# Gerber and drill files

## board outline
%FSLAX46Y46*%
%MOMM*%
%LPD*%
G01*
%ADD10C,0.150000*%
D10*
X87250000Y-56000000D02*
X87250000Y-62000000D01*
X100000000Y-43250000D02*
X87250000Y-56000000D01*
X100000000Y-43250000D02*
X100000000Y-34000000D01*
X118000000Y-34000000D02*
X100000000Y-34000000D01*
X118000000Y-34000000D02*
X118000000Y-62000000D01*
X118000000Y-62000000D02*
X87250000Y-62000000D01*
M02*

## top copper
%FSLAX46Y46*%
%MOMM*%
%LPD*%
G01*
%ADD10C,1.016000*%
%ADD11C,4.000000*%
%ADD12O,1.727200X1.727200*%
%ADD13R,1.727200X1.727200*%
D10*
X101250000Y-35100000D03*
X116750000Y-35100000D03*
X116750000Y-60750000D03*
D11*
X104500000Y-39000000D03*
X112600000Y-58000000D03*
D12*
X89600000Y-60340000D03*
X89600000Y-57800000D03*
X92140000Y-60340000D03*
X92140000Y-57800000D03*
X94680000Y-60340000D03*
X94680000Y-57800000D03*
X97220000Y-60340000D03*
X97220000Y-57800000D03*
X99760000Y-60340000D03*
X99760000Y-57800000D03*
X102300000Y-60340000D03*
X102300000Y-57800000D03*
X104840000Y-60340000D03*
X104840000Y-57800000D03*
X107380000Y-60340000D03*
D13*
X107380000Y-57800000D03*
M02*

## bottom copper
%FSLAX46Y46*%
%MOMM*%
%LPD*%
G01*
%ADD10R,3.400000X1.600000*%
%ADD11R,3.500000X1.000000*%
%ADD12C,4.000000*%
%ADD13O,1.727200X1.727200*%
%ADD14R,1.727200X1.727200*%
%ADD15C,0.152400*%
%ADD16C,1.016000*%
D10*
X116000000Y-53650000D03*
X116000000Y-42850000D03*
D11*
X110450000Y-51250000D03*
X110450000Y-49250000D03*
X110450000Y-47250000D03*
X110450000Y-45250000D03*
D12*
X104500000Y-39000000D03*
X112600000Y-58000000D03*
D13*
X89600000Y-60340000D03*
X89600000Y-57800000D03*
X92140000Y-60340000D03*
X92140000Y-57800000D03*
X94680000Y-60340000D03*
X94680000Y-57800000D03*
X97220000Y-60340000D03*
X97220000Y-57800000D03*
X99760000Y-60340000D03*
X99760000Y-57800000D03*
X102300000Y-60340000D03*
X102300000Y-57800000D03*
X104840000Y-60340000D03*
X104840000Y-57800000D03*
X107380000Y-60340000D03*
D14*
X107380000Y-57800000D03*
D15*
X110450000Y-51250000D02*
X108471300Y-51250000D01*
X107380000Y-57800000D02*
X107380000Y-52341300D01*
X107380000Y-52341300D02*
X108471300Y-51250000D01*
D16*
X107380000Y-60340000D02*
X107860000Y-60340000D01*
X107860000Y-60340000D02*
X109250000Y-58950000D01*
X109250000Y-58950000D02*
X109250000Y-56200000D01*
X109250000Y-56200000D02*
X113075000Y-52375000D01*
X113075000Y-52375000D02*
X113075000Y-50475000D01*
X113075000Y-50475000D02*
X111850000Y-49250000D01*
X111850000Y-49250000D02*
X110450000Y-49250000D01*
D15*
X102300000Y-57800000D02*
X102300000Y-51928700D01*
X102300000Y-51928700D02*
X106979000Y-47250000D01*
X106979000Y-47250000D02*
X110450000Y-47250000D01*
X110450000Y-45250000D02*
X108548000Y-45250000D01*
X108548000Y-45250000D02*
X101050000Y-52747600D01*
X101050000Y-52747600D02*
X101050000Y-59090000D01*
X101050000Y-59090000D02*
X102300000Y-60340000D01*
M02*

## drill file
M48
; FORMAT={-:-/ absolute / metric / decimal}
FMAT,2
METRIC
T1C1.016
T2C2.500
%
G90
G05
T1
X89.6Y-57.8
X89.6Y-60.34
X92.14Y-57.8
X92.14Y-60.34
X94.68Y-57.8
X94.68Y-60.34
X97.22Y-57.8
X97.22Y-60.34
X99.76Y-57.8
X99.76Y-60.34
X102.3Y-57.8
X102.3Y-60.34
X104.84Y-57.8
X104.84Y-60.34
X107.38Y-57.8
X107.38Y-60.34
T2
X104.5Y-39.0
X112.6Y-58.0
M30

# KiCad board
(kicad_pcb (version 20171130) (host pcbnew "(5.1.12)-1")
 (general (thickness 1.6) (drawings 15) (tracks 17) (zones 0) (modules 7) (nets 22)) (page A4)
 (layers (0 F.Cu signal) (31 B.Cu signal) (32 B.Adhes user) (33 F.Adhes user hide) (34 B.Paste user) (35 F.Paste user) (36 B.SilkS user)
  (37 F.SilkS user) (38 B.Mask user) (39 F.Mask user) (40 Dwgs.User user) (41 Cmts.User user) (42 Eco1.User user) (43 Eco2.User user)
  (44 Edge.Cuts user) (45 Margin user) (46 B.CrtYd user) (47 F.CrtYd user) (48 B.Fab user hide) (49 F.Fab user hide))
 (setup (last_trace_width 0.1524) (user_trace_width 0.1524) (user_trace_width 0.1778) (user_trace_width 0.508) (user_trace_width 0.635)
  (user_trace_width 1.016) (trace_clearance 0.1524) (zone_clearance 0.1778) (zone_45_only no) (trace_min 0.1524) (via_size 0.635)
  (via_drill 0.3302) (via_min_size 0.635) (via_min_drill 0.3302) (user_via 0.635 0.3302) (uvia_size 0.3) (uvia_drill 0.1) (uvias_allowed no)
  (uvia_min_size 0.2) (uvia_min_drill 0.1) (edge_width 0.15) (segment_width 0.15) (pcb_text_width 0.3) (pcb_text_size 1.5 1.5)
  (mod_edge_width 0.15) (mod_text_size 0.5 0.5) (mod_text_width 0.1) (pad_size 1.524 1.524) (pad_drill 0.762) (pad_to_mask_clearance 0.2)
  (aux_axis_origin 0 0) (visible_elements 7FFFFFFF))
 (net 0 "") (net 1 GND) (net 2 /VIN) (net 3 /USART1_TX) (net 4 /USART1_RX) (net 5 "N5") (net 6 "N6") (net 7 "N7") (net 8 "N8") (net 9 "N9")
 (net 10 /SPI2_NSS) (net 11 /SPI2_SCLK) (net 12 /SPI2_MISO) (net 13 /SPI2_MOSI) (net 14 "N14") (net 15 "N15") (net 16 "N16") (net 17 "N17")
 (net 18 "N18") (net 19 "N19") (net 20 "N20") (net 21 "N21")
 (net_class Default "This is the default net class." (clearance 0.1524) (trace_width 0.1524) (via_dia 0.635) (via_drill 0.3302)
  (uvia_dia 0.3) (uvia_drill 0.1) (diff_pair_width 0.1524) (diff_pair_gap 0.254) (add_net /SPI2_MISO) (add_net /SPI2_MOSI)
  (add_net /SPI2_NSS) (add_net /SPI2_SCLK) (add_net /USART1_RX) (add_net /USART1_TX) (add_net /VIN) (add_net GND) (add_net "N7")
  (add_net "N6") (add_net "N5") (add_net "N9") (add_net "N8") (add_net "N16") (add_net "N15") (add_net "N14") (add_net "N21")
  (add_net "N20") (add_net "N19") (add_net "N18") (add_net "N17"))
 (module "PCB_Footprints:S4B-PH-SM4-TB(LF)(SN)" (layer B.Cu) (at 113.225 48.25 270)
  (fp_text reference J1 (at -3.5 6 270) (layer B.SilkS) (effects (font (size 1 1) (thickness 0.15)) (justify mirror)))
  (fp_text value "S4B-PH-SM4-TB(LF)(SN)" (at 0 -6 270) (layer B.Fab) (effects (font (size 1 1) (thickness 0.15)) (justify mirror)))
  (pad "" smd rect (at 5.4 -2.775 270) (size 1.6 3.4) (layers B.Cu B.Paste B.Mask))
  (pad "" smd rect (at -5.4 -2.775 270) (size 1.6 3.4) (layers B.Cu B.Paste B.Mask))
  (pad 4 smd rect (at 3 2.775 270) (size 1 3.5) (layers B.Cu B.Paste B.Mask) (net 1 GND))
  (pad 3 smd rect (at 1 2.775 270) (size 1 3.5) (layers B.Cu B.Paste B.Mask) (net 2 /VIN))
  (pad 2 smd rect (at -1 2.775 270) (size 1 3.5) (layers B.Cu B.Paste B.Mask) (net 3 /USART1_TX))
  (pad 1 smd rect (at -3 2.775 270) (size 1 3.5) (layers B.Cu B.Paste B.Mask) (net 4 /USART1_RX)))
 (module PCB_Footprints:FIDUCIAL (layer F.Cu) (at 101.25 35.1) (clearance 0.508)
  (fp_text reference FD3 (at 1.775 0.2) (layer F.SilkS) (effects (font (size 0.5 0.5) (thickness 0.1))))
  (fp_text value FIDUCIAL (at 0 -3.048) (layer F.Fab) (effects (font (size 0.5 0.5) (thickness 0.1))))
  (pad 1 smd circle (at 0 0) (size 1.016 1.016) (layers F.Cu F.Mask) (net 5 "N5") (solder_mask_margin 0.508)))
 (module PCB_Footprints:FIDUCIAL (layer F.Cu) (at 116.75 35.1) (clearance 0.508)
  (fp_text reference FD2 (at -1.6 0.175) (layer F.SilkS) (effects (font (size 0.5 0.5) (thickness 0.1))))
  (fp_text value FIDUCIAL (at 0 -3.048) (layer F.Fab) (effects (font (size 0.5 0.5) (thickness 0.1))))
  (pad 1 smd circle (at 0 0) (size 1.016 1.016) (layers F.Cu F.Mask) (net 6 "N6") (solder_mask_margin 0.508)))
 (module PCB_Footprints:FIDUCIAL (layer F.Cu) (at 116.75 60.75) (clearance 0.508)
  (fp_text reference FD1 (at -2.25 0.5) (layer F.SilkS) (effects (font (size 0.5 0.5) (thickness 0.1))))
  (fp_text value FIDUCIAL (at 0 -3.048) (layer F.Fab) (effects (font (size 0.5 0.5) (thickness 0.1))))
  (pad 1 smd circle (at 0 0) (size 1.016 1.016) (layers F.Cu F.Mask) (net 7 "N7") (solder_mask_margin 0.508)))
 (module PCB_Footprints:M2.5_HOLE (layer F.Cu) (at 104.5 39)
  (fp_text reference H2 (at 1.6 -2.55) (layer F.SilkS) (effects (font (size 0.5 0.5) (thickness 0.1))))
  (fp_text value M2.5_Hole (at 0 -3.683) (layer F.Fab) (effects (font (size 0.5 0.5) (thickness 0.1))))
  (pad 1 thru_hole circle (at 0 0) (size 4 4) (drill 2.5) (layers *.Cu *.Mask) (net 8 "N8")))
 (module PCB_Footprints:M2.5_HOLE (layer F.Cu) (at 112.6 58 90)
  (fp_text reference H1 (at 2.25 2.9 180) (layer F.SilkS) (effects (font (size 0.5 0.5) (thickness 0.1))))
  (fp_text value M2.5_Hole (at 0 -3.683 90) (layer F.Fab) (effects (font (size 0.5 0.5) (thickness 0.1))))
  (pad 1 thru_hole circle (at 0 0 90) (size 4 4) (drill 2.5) (layers *.Cu *.Mask) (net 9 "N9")))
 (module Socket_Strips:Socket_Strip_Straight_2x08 (layer B.Cu) (at 107.38 57.8 180)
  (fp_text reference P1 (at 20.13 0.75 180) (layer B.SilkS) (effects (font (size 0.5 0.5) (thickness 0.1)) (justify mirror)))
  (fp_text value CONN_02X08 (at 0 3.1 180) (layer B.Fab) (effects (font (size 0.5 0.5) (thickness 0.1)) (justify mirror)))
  (pad 16 thru_hole oval (at 17.78 -2.54 180) (size 1.7272 1.7272) (drill 1.016) (layers *.Cu *.Mask) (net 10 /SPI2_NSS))
  (pad 15 thru_hole oval (at 17.78 0 180) (size 1.7272 1.7272) (drill 1.016) (layers *.Cu *.Mask) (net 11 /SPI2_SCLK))
  (pad 14 thru_hole oval (at 15.24 -2.54 180) (size 1.7272 1.7272) (drill 1.016) (layers *.Cu *.Mask) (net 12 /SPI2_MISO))
  (pad 13 thru_hole oval (at 15.24 0 180) (size 1.7272 1.7272) (drill 1.016) (layers *.Cu *.Mask) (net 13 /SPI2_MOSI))
  (pad 12 thru_hole oval (at 12.7 -2.54 180) (size 1.7272 1.7272) (drill 1.016) (layers *.Cu *.Mask) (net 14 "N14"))
  (pad 11 thru_hole oval (at 12.7 0 180) (size 1.7272 1.7272) (drill 1.016) (layers *.Cu *.Mask) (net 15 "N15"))
  (pad 10 thru_hole oval (at 10.16 -2.54 180) (size 1.7272 1.7272) (drill 1.016) (layers *.Cu *.Mask) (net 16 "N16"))
  (pad 9 thru_hole oval (at 10.16 0 180) (size 1.7272 1.7272) (drill 1.016) (layers *.Cu *.Mask) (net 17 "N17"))
  (pad 8 thru_hole oval (at 7.62 -2.54 180) (size 1.7272 1.7272) (drill 1.016) (layers *.Cu *.Mask) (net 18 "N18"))
  (pad 7 thru_hole oval (at 7.62 0 180) (size 1.7272 1.7272) (drill 1.016) (layers *.Cu *.Mask) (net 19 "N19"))
  (pad 6 thru_hole oval (at 5.08 -2.54 180) (size 1.7272 1.7272) (drill 1.016) (layers *.Cu *.Mask) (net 4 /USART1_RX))
  (pad 5 thru_hole oval (at 5.08 0 180) (size 1.7272 1.7272) (drill 1.016) (layers *.Cu *.Mask) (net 3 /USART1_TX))
  (pad 4 thru_hole oval (at 2.54 -2.54 180) (size 1.7272 1.7272) (drill 1.016) (layers *.Cu *.Mask) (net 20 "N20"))
  (pad 3 thru_hole oval (at 2.54 0 180) (size 1.7272 1.7272) (drill 1.016) (layers *.Cu *.Mask) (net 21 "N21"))
  (pad 2 thru_hole oval (at 0 -2.54 180) (size 1.7272 1.7272) (drill 1.016) (layers *.Cu *.Mask) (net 2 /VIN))
  (pad 1 thru_hole rect (at 0 0 180) (size 1.7272 1.7272) (drill 1.016) (layers *.Cu *.Mask) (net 1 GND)))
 (gr_line (start 87.25 56) (end 87.25 62) (layer Edge.Cuts) (width 0.15))
 (gr_line (start 100 43.25) (end 87.25 56) (layer Edge.Cuts) (width 0.15))
 (gr_line (start 100 43.25) (end 100 34) (layer Edge.Cuts) (width 0.15))
 (gr_line (start 118 34) (end 100 34) (layer Edge.Cuts) (width 0.15))
 (gr_line (start 118 34) (end 118 62) (layer Edge.Cuts) (width 0.15))
 (gr_line (start 118 62) (end 87.25 62) (layer Edge.Cuts) (width 0.15))
 (segment (start 110.45 51.25) (end 108.4713 51.25) (width 0.1524) (layer B.Cu) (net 1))
 (segment (start 107.38 57.8) (end 107.38 52.3413) (width 0.1524) (layer B.Cu) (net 1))
 (segment (start 107.38 52.3413) (end 108.4713 51.25) (width 0.1524) (layer B.Cu) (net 1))
 (segment (start 107.38 60.34) (end 107.86 60.34) (width 1.016) (layer B.Cu) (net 2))
 (segment (start 107.86 60.34) (end 109.25 58.95) (width 1.016) (layer B.Cu) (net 2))
 (segment (start 109.25 58.95) (end 109.25 56.2) (width 1.016) (layer B.Cu) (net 2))
 (segment (start 109.25 56.2) (end 113.075 52.375) (width 1.016) (layer B.Cu) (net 2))
 (segment (start 113.075 52.375) (end 113.075 50.475) (width 1.016) (layer B.Cu) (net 2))
 (segment (start 113.075 50.475) (end 111.85 49.25) (width 1.016) (layer B.Cu) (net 2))
 (segment (start 111.85 49.25) (end 110.45 49.25) (width 1.016) (layer B.Cu) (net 2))
 (segment (start 102.3 57.8) (end 102.3 51.9287) (width 0.1524) (layer B.Cu) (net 3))
 (segment (start 102.3 51.9287) (end 106.979 47.25) (width 0.1524) (layer B.Cu) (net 3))
 (segment (start 106.979 47.25) (end 110.45 47.25) (width 0.1524) (layer B.Cu) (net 3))
 (segment (start 110.45 45.25) (end 108.548 45.25) (width 0.1524) (layer B.Cu) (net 4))
 (segment (start 108.548 45.25) (end 101.05 52.7476) (width 0.1524) (layer B.Cu) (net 4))
 (segment (start 101.05 52.7476) (end 101.05 59.09) (width 0.1524) (layer B.Cu) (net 4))
 (segment (start 101.05 59.09) (end 102.3 60.34) (width 0.1524) (layer B.Cu) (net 4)))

